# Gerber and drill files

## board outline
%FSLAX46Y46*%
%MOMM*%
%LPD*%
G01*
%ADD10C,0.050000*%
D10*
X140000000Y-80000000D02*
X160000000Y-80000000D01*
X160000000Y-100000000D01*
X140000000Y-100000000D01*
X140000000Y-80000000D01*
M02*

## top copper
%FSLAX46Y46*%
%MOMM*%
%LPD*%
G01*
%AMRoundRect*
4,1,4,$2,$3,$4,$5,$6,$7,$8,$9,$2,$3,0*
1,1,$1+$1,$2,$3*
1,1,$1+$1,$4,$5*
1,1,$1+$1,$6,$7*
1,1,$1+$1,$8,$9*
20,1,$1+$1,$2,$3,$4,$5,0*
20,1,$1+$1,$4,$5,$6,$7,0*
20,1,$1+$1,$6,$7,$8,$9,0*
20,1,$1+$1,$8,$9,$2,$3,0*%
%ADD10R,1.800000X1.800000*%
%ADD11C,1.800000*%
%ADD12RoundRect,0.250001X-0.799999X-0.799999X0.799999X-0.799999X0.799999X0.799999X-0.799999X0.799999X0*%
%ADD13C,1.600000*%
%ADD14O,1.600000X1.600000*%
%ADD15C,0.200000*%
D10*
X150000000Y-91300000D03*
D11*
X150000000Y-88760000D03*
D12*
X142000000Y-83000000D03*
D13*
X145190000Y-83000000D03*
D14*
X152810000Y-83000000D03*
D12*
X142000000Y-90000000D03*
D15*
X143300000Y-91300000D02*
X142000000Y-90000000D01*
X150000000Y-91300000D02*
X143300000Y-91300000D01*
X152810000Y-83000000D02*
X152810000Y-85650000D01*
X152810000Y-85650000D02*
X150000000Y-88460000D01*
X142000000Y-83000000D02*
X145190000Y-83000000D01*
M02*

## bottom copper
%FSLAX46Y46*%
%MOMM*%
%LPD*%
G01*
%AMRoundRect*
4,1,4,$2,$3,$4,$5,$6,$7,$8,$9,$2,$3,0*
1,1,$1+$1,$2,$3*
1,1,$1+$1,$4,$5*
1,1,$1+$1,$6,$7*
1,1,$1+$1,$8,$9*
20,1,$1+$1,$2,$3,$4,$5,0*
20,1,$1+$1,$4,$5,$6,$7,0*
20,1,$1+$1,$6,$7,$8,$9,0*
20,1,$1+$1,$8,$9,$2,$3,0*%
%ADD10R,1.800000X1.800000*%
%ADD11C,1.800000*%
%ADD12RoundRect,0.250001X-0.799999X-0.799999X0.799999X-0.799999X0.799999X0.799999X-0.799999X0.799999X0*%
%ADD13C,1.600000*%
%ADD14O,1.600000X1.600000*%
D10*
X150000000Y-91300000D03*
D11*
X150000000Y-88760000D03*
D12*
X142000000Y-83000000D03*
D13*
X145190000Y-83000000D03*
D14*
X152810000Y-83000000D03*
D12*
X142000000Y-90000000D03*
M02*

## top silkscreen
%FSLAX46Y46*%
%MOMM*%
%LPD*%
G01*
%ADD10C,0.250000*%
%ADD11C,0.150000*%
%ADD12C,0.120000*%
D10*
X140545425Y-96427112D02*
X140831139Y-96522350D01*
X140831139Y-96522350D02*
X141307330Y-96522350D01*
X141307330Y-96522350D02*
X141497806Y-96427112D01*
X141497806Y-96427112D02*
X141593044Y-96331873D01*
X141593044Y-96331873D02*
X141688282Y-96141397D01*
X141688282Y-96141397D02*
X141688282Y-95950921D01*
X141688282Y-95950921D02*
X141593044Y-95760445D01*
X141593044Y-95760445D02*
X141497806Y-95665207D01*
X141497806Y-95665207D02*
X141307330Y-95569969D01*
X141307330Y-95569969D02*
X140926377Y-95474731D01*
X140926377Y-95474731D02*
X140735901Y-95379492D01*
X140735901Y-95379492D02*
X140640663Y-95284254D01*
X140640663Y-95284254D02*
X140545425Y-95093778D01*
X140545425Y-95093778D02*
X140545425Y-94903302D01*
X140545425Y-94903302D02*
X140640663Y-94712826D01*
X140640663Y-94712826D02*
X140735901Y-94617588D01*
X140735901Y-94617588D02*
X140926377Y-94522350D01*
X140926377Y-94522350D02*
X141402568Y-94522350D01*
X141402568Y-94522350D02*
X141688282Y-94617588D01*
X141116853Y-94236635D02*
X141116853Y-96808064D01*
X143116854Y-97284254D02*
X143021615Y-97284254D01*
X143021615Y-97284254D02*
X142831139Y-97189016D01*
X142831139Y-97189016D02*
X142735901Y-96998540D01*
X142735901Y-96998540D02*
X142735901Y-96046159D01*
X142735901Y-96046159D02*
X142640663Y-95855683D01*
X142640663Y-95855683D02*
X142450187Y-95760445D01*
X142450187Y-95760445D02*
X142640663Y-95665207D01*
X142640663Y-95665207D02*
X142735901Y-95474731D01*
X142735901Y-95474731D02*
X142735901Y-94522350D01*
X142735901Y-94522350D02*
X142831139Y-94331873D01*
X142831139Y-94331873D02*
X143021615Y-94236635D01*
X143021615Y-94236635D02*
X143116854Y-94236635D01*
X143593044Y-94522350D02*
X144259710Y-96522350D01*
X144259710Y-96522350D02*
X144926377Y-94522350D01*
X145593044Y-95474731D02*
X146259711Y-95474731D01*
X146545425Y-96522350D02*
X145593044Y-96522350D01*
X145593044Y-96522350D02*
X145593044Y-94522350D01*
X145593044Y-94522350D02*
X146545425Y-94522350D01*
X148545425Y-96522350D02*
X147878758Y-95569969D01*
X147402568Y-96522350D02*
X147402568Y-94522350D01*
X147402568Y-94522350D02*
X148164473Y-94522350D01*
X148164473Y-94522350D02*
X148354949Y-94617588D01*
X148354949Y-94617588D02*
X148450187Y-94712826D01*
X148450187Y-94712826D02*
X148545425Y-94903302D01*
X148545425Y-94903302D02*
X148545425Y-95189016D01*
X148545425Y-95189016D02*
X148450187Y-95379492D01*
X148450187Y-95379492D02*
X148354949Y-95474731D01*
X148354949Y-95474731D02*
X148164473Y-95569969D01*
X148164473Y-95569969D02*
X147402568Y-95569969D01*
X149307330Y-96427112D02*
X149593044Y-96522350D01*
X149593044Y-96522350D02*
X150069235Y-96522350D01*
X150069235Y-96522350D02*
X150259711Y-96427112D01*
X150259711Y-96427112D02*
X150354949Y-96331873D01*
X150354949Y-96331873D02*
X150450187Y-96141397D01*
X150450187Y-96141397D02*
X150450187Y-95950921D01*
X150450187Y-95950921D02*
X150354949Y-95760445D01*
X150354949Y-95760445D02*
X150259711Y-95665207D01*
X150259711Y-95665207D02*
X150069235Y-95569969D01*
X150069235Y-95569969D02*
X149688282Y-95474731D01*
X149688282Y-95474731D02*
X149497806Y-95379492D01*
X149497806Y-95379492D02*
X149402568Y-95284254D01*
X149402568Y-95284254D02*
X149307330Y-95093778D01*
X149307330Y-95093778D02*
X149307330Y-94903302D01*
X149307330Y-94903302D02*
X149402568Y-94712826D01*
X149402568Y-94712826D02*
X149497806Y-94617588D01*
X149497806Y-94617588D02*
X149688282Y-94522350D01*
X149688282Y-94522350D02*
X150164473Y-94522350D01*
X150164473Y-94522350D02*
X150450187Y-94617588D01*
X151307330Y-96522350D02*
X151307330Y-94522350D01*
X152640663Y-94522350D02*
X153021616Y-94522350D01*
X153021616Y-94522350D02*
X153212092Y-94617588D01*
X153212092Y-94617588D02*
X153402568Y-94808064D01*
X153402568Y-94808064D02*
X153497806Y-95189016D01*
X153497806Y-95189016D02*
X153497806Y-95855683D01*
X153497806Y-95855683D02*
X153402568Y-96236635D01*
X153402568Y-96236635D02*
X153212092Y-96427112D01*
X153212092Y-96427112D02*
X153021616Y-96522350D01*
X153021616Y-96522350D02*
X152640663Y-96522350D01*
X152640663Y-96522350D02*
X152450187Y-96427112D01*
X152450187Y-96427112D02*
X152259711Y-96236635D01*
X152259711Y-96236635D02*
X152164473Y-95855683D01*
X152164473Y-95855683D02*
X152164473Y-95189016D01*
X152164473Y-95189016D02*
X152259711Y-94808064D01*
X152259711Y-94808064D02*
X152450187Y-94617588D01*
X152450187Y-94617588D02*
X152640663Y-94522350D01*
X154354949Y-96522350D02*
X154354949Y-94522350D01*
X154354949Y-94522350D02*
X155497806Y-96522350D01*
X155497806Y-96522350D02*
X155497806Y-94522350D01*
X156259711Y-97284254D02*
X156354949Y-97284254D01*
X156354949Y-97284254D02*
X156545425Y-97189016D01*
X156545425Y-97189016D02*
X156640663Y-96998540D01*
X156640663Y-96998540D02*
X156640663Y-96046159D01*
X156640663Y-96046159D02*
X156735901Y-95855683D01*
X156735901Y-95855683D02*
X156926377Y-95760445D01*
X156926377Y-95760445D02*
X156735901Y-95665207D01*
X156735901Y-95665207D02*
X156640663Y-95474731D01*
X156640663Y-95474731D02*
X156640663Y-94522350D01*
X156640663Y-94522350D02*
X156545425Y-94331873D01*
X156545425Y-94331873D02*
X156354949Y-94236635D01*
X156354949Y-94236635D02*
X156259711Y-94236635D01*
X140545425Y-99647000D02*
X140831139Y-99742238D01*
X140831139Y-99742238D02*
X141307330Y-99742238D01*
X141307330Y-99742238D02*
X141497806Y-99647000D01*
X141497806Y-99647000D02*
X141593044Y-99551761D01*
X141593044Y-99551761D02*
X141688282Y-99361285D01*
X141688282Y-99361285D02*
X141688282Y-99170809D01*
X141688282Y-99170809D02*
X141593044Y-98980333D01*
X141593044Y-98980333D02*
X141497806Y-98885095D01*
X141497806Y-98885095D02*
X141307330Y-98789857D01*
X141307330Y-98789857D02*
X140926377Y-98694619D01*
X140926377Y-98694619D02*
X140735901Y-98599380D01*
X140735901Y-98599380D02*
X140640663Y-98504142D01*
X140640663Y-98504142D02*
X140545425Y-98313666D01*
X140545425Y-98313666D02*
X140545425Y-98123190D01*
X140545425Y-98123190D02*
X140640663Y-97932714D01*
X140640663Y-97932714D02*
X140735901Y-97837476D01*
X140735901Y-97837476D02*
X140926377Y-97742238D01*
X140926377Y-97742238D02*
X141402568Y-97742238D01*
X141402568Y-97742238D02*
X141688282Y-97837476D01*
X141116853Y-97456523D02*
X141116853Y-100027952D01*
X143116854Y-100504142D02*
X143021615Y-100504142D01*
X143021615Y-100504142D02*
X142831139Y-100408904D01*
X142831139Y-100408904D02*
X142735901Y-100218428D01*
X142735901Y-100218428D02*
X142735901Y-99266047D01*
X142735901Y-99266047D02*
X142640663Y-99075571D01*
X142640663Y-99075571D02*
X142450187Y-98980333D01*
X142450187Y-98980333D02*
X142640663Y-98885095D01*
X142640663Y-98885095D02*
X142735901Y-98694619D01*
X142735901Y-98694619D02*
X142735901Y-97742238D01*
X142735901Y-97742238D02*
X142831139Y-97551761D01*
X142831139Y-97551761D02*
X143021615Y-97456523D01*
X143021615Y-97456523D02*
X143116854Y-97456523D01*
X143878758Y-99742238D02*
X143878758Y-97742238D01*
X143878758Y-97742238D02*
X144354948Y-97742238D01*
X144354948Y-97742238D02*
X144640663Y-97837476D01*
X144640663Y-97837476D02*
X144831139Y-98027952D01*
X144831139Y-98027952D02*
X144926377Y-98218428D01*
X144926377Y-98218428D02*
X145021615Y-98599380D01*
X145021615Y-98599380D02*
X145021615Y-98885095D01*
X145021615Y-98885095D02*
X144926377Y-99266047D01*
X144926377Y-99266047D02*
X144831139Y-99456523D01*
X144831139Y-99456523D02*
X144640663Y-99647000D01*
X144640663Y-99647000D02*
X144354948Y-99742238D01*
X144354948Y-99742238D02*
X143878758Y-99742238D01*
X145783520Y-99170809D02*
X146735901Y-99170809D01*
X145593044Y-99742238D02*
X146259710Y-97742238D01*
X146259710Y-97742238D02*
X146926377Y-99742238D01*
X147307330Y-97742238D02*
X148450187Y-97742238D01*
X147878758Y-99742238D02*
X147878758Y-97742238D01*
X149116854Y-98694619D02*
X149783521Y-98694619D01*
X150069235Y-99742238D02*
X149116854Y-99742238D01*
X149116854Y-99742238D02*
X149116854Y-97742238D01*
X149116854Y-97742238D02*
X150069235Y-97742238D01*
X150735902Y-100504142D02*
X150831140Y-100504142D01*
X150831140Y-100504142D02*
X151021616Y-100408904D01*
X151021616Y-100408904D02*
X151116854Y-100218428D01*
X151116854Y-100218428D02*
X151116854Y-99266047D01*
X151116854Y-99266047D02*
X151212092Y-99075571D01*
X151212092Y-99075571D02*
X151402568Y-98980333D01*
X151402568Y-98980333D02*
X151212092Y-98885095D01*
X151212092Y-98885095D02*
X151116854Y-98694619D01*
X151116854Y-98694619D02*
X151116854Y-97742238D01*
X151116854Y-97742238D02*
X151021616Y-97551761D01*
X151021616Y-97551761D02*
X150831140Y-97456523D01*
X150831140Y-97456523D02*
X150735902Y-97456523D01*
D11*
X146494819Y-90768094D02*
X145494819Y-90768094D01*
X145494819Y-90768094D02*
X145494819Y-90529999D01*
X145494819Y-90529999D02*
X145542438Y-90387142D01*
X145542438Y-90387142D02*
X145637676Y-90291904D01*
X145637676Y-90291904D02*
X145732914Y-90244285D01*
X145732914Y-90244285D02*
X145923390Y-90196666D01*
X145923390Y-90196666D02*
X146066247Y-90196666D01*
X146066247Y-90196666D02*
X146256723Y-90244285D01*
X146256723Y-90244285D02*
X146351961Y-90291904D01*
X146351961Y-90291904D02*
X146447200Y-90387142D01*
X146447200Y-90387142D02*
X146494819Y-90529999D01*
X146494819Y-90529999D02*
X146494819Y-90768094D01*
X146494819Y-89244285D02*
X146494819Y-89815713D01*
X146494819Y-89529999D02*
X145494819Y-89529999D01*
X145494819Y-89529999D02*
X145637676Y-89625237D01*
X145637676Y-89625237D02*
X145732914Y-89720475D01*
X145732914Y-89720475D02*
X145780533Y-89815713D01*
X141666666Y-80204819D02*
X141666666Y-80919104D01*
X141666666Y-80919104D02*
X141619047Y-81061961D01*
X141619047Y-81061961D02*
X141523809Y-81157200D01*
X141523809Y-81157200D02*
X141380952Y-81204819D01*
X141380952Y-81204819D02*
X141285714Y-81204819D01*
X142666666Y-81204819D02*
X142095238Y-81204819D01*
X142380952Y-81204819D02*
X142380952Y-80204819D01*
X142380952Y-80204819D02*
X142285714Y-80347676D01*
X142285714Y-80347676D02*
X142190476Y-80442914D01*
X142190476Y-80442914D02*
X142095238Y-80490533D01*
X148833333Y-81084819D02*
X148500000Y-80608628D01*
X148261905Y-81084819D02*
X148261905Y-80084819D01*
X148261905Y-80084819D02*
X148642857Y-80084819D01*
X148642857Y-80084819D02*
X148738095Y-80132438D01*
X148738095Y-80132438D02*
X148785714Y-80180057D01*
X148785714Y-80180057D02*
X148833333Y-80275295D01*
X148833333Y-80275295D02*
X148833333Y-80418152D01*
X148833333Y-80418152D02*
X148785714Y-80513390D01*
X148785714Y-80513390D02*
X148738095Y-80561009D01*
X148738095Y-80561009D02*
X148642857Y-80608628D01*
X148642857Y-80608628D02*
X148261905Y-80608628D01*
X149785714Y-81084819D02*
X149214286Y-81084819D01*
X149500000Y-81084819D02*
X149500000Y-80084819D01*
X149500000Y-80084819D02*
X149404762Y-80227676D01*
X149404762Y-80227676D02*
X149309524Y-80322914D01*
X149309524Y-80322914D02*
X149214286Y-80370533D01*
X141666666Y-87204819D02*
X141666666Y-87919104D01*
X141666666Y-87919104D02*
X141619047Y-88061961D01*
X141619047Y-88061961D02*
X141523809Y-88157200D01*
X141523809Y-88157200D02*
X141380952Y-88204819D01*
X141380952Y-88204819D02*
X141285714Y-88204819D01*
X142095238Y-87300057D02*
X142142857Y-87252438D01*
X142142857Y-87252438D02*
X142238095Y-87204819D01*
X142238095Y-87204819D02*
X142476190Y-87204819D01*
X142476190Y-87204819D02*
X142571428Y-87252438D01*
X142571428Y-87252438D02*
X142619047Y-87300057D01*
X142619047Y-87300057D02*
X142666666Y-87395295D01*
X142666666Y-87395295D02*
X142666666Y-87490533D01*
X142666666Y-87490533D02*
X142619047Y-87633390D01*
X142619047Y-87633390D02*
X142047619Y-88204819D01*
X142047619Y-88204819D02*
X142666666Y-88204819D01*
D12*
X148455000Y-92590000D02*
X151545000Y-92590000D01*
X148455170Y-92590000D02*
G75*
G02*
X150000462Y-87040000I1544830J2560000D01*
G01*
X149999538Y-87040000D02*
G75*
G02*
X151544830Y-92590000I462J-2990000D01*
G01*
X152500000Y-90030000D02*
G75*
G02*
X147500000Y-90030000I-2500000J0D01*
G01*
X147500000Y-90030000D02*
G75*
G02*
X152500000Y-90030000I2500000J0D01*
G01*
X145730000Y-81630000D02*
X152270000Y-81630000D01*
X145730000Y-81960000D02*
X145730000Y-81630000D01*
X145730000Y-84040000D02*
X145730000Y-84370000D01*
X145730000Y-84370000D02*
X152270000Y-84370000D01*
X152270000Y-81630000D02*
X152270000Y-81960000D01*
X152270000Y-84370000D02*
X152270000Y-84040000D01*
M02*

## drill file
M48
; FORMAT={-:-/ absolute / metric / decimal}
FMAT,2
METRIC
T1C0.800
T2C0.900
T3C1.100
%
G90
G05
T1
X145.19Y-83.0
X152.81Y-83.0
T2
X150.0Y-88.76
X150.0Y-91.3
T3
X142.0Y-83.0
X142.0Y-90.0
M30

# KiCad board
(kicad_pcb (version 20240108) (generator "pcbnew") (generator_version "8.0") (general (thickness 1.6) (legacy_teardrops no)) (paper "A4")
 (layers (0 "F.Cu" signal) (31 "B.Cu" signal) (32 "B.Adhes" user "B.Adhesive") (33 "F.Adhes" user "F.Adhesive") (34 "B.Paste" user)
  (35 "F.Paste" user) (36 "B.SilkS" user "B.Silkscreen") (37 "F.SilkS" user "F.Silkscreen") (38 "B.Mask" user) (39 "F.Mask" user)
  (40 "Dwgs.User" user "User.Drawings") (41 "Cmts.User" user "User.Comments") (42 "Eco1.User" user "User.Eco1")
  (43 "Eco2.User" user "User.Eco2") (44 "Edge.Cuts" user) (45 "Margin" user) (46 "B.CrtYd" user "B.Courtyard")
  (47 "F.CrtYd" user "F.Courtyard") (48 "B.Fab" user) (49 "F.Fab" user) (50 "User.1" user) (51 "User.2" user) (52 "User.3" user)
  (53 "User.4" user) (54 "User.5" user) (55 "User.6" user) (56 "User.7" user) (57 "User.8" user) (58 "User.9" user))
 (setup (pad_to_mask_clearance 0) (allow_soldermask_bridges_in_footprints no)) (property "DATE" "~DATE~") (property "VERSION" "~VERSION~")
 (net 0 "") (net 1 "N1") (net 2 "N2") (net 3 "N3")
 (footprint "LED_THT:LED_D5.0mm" (layer "F.Cu") (at 150 91.3 90)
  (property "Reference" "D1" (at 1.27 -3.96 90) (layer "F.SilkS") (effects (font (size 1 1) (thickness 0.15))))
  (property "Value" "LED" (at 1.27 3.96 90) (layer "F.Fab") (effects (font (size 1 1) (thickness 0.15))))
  (fp_line (start -1.29 -1.545) (end -1.29 1.545) (stroke (width 0.12) (type solid)) (layer "F.SilkS"))
  (fp_arc (start -1.29 -1.54483) (mid 2.072002 -2.880433) (end 4.26 0.000462) (stroke (width 0.12) (type solid)) (layer "F.SilkS"))
  (fp_arc (start 4.26 -0.000462) (mid 2.072002 2.880433) (end -1.29 1.54483) (stroke (width 0.12) (type solid)) (layer "F.SilkS"))
  (fp_circle (center 1.27 0) (end 3.77 0) (stroke (width 0.12) (type solid)) (fill none) (layer "F.SilkS"))
  (pad "1" thru_hole rect (at 0 0 90) (size 1.8 1.8) (drill 0.9) (layers "*.Cu" "*.Mask") (remove_unused_layers no) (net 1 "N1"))
  (pad "2" thru_hole circle (at 2.54 0 90) (size 1.8 1.8) (drill 0.9) (layers "*.Cu" "*.Mask") (remove_unused_layers no) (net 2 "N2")))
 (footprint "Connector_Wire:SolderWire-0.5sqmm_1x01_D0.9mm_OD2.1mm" (layer "F.Cu") (at 142 83)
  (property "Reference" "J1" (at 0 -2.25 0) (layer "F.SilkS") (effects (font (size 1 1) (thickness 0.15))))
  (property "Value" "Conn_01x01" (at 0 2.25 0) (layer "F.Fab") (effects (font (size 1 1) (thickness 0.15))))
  (pad "1" thru_hole roundrect (at 0 0) (size 2.1 2.1) (drill 1.1) (layers "*.Cu" "*.Mask") (remove_unused_layers no)
   (roundrect_rratio 0.119048) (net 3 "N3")))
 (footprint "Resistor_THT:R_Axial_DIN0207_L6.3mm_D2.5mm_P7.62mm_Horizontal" (layer "F.Cu") (at 145.19 83)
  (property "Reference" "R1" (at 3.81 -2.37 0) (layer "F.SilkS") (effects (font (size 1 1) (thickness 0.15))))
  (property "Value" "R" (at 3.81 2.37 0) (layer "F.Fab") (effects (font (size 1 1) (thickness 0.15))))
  (fp_line (start 0.54 -1.37) (end 7.08 -1.37) (stroke (width 0.12) (type solid)) (layer "F.SilkS"))
  (fp_line (start 0.54 -1.04) (end 0.54 -1.37) (stroke (width 0.12) (type solid)) (layer "F.SilkS"))
  (fp_line (start 0.54 1.04) (end 0.54 1.37) (stroke (width 0.12) (type solid)) (layer "F.SilkS"))
  (fp_line (start 0.54 1.37) (end 7.08 1.37) (stroke (width 0.12) (type solid)) (layer "F.SilkS"))
  (fp_line (start 7.08 -1.37) (end 7.08 -1.04) (stroke (width 0.12) (type solid)) (layer "F.SilkS"))
  (fp_line (start 7.08 1.37) (end 7.08 1.04) (stroke (width 0.12) (type solid)) (layer "F.SilkS"))
  (pad "1" thru_hole circle (at 0 0) (size 1.6 1.6) (drill 0.8) (layers "*.Cu" "*.Mask") (remove_unused_layers no) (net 3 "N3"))
  (pad "2" thru_hole oval (at 7.62 0) (size 1.6 1.6) (drill 0.8) (layers "*.Cu" "*.Mask") (remove_unused_layers no) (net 2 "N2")))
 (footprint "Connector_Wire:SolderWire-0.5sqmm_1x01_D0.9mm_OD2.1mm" (layer "F.Cu") (at 142 90)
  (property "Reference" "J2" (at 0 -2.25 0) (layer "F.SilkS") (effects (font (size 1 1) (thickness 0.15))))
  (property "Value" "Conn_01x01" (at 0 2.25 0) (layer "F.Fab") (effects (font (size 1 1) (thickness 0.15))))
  (pad "1" thru_hole roundrect (at 0 0) (size 2.1 2.1) (drill 1.1) (layers "*.Cu" "*.Mask") (remove_unused_layers no)
   (roundrect_rratio 0.119048) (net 1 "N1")))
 (gr_rect (start 140 80) (end 160 100) (stroke (width 0.05) (type default)) (fill none) (layer "Edge.Cuts"))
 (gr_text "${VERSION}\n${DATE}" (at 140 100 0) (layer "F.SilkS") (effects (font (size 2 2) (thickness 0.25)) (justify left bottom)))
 (segment (start 143.3 91.3) (end 142 90) (width 0.2) (layer "F.Cu") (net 1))
 (segment (start 150 91.3) (end 143.3 91.3) (width 0.2) (layer "F.Cu") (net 1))
 (segment (start 152.81 83) (end 152.81 85.65) (width 0.2) (layer "F.Cu") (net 2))
 (segment (start 152.81 85.65) (end 150 88.46) (width 0.2) (layer "F.Cu") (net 2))
 (segment (start 142 83) (end 145.19 83) (width 0.2) (layer "F.Cu") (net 3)))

